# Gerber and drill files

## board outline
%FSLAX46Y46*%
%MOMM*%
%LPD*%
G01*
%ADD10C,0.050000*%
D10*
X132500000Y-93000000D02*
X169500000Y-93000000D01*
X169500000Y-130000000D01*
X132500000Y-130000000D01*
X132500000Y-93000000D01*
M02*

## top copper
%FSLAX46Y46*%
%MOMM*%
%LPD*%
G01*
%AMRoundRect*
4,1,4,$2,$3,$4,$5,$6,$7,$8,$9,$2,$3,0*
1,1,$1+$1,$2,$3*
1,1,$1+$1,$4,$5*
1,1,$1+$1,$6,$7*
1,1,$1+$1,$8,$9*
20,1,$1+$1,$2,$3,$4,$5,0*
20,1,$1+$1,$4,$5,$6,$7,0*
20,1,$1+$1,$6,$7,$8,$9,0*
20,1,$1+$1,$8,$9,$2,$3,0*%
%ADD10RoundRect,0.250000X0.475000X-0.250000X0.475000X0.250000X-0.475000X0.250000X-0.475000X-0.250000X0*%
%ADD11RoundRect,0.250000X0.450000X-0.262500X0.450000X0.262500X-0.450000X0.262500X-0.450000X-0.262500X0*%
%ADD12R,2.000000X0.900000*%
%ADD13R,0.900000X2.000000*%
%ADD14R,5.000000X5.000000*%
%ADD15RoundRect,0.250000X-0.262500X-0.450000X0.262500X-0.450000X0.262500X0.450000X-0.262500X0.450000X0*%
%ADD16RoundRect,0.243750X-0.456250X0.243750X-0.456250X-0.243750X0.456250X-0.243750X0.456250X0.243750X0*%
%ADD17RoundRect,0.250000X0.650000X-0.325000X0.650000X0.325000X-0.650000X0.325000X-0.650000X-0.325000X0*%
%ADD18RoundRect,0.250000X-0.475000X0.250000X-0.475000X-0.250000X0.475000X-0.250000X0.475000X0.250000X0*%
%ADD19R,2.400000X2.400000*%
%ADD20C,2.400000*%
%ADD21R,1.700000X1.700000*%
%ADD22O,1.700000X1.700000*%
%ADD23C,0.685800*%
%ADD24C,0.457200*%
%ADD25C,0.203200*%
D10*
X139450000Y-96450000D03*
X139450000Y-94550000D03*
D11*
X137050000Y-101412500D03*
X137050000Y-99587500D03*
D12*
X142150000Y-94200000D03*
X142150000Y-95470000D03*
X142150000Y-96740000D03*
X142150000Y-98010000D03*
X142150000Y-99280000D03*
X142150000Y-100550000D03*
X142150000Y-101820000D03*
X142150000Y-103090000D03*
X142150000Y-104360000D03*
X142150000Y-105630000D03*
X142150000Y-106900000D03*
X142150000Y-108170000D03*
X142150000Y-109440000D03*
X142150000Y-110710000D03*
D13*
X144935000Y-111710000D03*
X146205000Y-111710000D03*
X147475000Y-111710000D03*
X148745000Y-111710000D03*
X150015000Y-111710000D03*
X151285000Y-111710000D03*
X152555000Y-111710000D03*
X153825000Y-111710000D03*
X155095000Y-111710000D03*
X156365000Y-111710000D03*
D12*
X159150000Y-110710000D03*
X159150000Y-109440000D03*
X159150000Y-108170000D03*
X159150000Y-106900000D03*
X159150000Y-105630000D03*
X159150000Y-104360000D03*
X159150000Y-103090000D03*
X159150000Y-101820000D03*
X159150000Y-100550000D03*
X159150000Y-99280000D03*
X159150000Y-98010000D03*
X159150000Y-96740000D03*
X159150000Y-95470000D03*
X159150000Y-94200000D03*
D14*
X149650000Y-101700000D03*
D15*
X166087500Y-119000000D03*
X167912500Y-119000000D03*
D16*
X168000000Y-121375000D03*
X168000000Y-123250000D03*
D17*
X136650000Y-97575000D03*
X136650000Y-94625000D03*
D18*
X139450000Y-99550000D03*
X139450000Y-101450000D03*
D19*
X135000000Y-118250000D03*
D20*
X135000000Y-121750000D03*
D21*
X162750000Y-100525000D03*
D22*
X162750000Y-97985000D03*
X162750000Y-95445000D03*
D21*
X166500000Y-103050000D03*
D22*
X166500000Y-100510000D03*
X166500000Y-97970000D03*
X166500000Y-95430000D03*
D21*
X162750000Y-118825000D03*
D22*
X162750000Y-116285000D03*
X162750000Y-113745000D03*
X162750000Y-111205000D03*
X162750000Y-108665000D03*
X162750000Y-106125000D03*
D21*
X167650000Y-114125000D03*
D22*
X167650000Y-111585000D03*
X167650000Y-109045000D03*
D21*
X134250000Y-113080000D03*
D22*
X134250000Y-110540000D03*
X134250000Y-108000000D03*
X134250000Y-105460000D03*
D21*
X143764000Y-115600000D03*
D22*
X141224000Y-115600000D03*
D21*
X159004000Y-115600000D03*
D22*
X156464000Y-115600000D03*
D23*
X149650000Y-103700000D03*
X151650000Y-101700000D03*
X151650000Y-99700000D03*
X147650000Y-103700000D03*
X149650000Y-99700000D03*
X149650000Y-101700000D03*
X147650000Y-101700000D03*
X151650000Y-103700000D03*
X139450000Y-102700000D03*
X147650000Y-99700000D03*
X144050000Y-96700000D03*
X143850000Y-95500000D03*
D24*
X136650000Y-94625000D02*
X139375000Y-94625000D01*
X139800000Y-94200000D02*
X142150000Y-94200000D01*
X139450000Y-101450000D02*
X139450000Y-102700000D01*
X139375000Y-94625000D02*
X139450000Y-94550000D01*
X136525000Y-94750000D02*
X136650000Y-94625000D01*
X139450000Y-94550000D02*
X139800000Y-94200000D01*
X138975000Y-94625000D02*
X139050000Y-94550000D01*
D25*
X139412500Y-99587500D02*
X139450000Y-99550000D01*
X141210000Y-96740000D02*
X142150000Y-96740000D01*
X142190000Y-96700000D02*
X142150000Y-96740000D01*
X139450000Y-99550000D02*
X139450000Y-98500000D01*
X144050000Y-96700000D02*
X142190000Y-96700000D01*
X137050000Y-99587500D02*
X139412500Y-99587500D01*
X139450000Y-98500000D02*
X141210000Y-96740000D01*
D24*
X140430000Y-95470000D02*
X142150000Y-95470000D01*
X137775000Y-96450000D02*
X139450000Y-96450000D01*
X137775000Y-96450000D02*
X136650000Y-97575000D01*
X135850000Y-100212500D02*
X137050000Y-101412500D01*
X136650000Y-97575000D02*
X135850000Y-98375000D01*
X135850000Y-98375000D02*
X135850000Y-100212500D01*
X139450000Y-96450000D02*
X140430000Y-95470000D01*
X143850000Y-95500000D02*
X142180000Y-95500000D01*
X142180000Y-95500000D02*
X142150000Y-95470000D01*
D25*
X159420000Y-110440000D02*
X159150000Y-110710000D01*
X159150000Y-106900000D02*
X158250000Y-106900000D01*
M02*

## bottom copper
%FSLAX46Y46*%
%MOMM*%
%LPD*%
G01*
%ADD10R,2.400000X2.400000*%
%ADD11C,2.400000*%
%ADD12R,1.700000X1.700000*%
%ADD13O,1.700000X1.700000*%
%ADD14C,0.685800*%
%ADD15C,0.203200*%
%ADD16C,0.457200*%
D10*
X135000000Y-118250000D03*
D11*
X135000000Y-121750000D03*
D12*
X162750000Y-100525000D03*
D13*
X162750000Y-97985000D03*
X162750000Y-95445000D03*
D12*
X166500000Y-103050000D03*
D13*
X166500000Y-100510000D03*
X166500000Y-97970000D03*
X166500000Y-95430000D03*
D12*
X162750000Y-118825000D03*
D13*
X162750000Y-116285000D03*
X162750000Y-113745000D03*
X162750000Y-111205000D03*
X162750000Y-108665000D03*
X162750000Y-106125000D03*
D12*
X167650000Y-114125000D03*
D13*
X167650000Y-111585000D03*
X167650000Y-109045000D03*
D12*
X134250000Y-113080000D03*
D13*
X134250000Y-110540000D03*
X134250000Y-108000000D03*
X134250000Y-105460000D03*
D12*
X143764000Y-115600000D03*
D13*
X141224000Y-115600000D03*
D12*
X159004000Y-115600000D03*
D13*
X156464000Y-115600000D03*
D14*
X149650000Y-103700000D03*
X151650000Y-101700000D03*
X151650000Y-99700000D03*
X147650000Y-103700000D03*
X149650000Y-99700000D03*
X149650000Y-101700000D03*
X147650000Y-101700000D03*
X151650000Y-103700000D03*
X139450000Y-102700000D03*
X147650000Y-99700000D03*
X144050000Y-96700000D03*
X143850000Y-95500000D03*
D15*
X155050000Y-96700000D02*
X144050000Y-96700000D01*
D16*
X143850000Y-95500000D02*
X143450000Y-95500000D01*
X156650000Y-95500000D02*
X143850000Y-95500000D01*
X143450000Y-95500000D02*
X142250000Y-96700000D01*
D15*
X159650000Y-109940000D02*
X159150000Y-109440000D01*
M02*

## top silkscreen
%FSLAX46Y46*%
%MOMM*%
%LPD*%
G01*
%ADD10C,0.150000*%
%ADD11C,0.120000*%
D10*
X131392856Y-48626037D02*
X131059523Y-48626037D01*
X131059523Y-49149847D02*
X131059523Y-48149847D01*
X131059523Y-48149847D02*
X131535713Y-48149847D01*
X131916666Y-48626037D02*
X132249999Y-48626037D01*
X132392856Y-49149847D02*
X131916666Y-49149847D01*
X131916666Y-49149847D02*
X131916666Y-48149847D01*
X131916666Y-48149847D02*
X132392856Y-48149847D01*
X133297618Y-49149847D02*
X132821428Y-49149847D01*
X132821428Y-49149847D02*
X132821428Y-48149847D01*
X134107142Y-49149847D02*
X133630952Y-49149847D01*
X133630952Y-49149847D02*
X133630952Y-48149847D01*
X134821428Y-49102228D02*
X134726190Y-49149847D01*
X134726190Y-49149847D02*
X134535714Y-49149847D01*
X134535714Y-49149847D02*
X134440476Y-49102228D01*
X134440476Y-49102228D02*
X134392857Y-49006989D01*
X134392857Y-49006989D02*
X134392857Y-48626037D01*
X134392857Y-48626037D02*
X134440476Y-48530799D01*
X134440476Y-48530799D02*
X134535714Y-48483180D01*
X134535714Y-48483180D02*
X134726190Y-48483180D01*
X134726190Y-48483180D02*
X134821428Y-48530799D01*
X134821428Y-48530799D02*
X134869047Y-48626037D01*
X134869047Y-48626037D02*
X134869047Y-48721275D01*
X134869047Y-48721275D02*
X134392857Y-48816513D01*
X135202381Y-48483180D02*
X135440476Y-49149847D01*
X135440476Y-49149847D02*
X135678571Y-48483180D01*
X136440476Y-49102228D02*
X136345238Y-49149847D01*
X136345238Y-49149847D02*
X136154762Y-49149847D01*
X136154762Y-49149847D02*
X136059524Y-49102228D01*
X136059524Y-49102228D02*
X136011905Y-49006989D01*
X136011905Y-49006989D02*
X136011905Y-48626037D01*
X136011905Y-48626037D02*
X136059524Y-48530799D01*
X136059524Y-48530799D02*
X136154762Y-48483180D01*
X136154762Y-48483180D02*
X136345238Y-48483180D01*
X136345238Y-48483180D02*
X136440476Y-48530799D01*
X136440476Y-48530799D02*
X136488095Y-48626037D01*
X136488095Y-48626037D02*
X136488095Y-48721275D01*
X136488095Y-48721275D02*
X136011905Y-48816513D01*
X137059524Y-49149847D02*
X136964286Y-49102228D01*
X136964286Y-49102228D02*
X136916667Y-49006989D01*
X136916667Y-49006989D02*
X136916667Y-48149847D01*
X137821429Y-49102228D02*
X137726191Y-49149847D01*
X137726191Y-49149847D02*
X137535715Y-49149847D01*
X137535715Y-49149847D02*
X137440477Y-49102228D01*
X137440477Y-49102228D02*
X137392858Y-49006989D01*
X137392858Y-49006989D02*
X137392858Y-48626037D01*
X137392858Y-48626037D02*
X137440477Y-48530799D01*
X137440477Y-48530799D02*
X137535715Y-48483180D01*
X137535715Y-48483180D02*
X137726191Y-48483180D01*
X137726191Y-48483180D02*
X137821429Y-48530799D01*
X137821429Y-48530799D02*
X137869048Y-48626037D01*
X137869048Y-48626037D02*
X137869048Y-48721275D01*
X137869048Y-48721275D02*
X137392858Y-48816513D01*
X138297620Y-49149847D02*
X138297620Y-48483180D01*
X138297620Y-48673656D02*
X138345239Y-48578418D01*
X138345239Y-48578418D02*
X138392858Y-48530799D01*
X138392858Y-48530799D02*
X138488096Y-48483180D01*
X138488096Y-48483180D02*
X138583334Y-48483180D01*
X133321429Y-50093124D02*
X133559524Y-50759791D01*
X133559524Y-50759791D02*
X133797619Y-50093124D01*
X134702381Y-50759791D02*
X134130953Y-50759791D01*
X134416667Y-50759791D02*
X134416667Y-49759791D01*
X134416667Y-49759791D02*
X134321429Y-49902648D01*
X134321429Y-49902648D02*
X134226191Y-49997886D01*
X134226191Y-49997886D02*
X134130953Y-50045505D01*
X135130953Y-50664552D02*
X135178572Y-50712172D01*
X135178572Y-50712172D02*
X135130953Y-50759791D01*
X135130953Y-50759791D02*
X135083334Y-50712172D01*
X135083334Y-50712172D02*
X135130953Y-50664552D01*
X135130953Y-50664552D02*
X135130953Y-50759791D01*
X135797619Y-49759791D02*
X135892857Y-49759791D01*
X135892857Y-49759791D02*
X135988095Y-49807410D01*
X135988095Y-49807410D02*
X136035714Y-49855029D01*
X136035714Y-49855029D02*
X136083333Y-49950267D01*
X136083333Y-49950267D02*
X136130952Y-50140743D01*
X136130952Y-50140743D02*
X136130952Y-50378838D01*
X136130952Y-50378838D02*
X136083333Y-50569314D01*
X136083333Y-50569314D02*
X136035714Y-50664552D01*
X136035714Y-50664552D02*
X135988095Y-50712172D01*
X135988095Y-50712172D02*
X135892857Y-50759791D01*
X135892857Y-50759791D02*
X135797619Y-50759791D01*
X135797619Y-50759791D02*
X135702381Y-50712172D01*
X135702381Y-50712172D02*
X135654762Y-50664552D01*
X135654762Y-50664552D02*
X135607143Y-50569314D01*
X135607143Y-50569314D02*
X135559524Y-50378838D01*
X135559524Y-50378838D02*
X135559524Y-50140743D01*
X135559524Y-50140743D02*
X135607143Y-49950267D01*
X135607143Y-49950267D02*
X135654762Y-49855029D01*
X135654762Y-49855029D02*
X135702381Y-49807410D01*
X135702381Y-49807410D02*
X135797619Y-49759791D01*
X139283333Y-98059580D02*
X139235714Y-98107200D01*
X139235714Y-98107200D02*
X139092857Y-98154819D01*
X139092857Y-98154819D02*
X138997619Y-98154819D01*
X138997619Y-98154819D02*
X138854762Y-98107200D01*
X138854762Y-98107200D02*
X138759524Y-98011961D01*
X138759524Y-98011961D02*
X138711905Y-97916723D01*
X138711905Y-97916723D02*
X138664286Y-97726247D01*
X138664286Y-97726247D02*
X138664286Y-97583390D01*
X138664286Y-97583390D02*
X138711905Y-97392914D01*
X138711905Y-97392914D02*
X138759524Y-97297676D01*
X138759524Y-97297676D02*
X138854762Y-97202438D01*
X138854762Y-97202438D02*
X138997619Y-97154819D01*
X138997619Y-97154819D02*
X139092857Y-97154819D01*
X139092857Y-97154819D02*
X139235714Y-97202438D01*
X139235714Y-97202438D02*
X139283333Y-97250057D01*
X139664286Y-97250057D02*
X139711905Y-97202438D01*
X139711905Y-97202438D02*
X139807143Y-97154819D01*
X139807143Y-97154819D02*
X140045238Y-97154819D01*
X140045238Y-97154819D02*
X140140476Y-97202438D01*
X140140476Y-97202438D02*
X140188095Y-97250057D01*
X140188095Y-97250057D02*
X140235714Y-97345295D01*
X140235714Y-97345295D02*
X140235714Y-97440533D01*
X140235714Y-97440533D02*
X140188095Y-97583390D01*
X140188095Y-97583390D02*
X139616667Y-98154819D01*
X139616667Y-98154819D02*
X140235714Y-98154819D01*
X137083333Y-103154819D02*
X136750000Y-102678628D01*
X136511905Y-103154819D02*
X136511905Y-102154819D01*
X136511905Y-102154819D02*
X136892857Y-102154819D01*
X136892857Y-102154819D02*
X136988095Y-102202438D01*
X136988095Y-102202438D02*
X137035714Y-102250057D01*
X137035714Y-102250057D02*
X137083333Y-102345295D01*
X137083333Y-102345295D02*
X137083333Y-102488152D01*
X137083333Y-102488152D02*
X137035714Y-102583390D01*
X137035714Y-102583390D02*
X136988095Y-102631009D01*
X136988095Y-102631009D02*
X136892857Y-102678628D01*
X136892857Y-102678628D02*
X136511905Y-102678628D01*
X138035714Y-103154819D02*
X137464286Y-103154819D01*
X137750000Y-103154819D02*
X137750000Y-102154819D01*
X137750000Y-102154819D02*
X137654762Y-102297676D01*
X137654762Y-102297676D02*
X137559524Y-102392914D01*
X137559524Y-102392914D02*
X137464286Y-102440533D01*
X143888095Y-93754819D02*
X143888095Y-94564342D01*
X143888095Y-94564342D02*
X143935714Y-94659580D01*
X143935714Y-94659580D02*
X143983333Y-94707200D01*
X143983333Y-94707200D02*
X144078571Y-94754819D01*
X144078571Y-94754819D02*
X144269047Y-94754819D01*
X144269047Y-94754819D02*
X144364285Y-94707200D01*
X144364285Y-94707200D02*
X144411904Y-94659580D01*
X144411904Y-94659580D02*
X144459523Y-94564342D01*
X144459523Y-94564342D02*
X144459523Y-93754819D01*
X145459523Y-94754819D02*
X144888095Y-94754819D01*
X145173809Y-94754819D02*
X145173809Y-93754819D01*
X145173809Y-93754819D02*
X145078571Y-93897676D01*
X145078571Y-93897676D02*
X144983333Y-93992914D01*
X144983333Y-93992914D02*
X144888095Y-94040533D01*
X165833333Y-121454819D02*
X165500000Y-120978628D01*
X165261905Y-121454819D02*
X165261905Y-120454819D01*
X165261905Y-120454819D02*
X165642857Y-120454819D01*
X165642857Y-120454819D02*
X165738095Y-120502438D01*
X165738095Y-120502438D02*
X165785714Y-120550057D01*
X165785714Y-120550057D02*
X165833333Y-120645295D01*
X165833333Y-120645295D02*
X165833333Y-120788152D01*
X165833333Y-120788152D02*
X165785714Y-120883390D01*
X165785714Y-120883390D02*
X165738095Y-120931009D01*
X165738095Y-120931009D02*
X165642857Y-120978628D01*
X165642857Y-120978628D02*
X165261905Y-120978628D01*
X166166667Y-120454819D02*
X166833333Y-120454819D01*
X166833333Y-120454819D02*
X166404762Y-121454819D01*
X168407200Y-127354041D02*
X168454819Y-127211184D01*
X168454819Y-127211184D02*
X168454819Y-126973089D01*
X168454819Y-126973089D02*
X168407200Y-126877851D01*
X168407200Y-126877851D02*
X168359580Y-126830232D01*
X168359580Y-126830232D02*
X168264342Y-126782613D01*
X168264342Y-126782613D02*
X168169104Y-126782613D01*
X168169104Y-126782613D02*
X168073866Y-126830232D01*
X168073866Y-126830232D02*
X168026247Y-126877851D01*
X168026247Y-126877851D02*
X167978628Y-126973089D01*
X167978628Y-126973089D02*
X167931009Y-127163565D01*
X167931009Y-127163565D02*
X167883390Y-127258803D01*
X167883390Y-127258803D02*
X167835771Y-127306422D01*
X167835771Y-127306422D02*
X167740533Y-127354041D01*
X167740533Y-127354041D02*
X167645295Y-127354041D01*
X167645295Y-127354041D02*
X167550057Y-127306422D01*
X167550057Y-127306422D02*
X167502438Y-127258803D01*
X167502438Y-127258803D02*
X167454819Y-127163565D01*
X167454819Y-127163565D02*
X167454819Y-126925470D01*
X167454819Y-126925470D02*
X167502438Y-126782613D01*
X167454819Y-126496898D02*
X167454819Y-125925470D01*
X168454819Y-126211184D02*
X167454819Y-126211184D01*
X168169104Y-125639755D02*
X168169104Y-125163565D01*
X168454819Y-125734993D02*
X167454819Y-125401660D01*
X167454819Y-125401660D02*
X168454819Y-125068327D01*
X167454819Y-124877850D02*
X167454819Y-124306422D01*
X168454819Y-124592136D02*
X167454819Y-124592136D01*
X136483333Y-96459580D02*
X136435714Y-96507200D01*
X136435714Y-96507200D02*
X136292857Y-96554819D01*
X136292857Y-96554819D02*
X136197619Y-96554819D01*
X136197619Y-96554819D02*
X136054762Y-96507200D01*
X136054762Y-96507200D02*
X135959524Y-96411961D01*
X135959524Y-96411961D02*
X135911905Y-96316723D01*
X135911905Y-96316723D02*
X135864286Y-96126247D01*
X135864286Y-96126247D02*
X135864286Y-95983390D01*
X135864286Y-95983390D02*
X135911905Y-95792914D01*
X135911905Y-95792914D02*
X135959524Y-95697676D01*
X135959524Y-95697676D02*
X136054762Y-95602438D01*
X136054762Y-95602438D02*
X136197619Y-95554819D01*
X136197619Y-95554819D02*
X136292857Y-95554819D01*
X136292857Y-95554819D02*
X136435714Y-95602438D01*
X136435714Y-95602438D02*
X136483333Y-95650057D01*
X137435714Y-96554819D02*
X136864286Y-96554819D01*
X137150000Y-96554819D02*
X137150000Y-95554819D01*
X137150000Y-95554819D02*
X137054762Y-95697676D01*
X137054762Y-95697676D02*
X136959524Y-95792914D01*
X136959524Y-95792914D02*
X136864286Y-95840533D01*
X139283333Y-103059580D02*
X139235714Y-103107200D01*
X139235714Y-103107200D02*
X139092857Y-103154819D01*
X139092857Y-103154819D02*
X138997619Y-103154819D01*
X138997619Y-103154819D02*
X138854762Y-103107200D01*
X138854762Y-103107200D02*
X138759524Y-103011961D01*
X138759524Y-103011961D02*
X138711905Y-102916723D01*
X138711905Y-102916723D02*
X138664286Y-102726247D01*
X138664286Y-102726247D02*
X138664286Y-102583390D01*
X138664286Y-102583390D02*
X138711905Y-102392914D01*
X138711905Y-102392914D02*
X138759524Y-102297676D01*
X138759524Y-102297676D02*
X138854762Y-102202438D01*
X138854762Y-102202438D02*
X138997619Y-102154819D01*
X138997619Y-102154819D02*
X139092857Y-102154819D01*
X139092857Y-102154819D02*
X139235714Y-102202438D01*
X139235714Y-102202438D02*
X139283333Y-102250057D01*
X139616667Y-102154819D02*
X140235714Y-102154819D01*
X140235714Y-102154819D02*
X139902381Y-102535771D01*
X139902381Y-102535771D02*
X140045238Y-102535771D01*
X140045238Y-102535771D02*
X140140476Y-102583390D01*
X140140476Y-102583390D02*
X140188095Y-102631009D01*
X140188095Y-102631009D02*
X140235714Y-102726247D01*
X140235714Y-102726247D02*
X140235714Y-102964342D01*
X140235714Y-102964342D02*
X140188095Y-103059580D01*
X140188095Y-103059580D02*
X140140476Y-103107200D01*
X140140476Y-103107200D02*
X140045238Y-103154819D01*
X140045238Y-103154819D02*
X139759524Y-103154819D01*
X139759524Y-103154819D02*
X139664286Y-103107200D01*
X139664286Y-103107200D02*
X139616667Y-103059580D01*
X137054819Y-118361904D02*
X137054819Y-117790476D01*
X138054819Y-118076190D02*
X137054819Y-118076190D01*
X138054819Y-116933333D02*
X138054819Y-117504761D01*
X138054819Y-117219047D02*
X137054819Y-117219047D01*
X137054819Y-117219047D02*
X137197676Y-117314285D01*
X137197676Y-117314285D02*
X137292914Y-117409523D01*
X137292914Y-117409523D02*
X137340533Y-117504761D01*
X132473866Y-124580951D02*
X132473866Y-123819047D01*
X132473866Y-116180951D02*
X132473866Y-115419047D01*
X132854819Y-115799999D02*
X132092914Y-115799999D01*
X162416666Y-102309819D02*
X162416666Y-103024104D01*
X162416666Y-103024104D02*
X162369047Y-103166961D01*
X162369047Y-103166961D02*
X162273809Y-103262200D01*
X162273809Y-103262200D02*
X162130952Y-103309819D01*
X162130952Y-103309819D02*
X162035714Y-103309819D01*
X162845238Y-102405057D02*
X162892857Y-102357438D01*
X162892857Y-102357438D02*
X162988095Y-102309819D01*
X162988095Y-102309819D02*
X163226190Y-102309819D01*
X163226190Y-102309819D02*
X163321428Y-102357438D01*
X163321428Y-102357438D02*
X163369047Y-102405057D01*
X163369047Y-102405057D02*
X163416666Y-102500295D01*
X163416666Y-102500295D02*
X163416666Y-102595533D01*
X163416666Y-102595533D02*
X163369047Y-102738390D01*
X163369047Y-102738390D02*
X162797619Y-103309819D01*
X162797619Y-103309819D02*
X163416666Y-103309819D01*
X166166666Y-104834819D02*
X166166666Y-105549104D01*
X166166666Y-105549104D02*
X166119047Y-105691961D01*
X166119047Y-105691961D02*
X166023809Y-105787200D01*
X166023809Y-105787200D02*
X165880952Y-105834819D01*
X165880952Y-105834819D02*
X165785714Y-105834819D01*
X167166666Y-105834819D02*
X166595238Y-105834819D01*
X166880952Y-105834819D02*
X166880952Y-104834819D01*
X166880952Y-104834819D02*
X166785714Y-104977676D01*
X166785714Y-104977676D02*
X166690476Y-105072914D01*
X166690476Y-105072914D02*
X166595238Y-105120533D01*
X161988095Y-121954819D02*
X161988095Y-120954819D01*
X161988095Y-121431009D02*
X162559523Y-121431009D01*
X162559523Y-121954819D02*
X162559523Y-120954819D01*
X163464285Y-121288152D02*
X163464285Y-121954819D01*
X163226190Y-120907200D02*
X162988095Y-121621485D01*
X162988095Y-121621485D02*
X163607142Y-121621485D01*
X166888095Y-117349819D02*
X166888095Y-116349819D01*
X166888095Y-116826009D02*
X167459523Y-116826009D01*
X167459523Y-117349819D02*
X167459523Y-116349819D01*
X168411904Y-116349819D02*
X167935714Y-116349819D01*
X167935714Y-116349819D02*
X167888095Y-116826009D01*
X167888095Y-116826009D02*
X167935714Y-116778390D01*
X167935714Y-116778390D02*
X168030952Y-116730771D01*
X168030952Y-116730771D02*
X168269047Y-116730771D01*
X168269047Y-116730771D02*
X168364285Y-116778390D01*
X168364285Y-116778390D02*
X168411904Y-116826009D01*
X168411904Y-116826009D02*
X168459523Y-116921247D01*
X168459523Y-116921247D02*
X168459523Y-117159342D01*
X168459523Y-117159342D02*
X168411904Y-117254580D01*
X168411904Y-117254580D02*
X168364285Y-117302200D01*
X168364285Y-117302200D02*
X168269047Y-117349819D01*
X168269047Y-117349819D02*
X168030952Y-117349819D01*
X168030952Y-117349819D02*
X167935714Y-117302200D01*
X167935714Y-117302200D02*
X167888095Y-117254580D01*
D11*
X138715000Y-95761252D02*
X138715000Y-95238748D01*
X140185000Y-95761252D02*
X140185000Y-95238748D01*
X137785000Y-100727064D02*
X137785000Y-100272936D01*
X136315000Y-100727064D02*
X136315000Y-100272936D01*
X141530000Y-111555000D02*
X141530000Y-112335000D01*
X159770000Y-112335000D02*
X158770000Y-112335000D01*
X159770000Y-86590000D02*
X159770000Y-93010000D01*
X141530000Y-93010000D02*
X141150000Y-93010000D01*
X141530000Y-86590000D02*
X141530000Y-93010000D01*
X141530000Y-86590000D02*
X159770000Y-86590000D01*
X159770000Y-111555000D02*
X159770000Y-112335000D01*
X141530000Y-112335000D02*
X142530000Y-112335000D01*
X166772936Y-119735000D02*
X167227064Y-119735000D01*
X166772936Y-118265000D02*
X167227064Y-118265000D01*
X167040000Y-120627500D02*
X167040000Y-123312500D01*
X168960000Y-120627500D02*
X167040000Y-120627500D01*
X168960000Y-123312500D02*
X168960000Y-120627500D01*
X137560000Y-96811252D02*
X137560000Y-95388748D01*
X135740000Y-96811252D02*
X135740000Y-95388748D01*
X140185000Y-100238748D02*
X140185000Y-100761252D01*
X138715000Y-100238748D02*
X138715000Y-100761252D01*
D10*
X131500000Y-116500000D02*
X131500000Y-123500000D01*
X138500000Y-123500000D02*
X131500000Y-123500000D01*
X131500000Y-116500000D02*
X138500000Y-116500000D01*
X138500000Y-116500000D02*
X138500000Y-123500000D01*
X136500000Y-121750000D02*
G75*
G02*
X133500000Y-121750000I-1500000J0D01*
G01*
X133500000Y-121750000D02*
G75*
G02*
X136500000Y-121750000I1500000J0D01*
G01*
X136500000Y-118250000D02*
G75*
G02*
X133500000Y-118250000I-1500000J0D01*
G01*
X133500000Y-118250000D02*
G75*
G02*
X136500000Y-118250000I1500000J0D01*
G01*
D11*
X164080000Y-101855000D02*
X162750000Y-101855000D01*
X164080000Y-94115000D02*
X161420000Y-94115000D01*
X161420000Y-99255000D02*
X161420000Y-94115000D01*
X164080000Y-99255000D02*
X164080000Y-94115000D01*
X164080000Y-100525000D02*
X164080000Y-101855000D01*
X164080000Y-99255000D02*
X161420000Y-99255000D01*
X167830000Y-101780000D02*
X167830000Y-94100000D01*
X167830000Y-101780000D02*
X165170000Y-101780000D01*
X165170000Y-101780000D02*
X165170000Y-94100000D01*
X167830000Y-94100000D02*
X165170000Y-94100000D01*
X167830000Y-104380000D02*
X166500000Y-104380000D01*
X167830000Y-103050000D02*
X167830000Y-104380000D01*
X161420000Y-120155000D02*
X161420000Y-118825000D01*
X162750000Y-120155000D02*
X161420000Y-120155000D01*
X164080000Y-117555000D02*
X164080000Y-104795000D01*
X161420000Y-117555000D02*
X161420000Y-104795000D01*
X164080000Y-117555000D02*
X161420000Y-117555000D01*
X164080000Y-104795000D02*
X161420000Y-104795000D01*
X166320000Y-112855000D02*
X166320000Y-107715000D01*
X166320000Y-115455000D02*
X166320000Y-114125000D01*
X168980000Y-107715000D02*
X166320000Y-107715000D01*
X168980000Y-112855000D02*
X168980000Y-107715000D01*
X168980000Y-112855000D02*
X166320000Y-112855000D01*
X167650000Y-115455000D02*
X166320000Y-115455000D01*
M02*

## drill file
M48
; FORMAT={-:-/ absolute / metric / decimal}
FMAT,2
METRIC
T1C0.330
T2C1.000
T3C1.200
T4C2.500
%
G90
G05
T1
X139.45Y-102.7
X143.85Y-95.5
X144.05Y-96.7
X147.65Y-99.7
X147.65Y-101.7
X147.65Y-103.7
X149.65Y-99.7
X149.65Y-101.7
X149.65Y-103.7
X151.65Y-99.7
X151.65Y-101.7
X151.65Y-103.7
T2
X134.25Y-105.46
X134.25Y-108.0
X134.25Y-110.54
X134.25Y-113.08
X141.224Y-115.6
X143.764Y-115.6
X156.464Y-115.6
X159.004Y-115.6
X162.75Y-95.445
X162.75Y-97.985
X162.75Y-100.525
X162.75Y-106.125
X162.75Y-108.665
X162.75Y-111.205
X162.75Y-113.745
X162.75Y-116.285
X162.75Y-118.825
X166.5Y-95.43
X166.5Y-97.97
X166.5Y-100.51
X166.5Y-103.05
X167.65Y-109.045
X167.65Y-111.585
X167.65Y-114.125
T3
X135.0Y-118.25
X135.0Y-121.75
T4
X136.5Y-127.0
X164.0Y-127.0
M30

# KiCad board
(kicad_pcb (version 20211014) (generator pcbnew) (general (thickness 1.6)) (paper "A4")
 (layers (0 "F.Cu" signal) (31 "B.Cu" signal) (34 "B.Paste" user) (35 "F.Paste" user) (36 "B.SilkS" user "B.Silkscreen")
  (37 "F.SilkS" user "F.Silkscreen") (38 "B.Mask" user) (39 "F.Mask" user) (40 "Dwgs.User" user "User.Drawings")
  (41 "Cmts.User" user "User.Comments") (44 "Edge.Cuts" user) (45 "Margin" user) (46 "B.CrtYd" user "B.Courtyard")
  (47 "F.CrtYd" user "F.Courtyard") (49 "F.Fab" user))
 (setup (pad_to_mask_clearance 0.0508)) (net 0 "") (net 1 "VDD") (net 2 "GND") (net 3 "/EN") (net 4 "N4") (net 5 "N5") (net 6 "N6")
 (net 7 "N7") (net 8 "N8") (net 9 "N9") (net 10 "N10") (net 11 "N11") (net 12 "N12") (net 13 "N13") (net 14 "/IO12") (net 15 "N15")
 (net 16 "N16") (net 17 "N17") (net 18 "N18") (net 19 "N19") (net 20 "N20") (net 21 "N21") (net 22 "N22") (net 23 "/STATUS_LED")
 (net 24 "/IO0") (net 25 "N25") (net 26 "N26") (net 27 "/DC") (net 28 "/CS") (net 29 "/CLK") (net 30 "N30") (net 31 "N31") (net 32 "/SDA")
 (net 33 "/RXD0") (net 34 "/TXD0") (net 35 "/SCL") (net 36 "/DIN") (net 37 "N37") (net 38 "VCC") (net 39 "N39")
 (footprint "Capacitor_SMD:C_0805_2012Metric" (layer "F.Cu") (at 139.45 95.5 90)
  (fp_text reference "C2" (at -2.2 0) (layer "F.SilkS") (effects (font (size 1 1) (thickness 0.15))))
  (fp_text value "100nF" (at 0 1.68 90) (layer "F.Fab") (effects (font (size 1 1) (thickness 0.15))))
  (fp_line (start -0.261252 -0.735) (end 0.261252 -0.735) (layer "F.SilkS") (width 0.12))
  (fp_line (start -0.261252 0.735) (end 0.261252 0.735) (layer "F.SilkS") (width 0.12))
  (pad "1" smd roundrect locked (at -0.95 0 90) (size 1 1.45) (layers "F.Cu" "F.Paste" "F.Mask") (roundrect_rratio 0.25) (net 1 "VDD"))
  (pad "2" smd roundrect locked (at 0.95 0 90) (size 1 1.45) (layers "F.Cu" "F.Paste" "F.Mask") (roundrect_rratio 0.25) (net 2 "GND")))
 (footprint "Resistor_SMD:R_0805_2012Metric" (layer "F.Cu") (at 137.05 100.5 90)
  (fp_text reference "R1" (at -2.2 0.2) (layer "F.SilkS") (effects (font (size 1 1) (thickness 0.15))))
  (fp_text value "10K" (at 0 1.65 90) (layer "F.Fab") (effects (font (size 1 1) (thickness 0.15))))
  (fp_line (start -0.227064 0.735) (end 0.227064 0.735) (layer "F.SilkS") (width 0.12))
  (fp_line (start -0.227064 -0.735) (end 0.227064 -0.735) (layer "F.SilkS") (width 0.12))
  (pad "1" smd roundrect locked (at -0.9125 0 90) (size 1.025 1.4) (layers "F.Cu" "F.Paste" "F.Mask") (roundrect_rratio 0.243902)
   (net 1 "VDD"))
  (pad "2" smd roundrect locked (at 0.9125 0 90) (size 1.025 1.4) (layers "F.Cu" "F.Paste" "F.Mask") (roundrect_rratio 0.243902)
   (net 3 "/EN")))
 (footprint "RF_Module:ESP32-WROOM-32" (layer "F.Cu") (at 150.65 102.455)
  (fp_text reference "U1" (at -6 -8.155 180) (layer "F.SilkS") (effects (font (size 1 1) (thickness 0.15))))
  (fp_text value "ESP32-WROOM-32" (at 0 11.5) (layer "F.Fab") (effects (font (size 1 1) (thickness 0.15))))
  (fp_line (start -9.12 9.1) (end -9.12 9.88) (layer "F.SilkS") (width 0.12))
  (fp_line (start 9.12 9.88) (end 8.12 9.88) (layer "F.SilkS") (width 0.12))
  (fp_line (start 9.12 -15.865) (end 9.12 -9.445) (layer "F.SilkS") (width 0.12))
  (fp_line (start -9.12 -9.445) (end -9.5 -9.445) (layer "F.SilkS") (width 0.12))
  (fp_line (start -9.12 -15.865) (end -9.12 -9.445) (layer "F.SilkS") (width 0.12))
  (fp_line (start -9.12 -15.865) (end 9.12 -15.865) (layer "F.SilkS") (width 0.12))
  (fp_line (start 9.12 9.1) (end 9.12 9.88) (layer "F.SilkS") (width 0.12))
  (fp_line (start -9.12 9.88) (end -8.12 9.88) (layer "F.SilkS") (width 0.12))
  (pad "1" smd rect locked (at -8.5 -8.255) (size 2 0.9) (layers "F.Cu" "F.Paste" "F.Mask") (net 2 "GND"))
  (pad "2" smd rect locked (at -8.5 -6.985) (size 2 0.9) (layers "F.Cu" "F.Paste" "F.Mask") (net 1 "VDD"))
  (pad "3" smd rect locked (at -8.5 -5.715) (size 2 0.9) (layers "F.Cu" "F.Paste" "F.Mask") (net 3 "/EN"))
  (pad "4" smd rect locked (at -8.5 -4.445) (size 2 0.9) (layers "F.Cu" "F.Paste" "F.Mask") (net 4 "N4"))
  (pad "5" smd rect locked (at -8.5 -3.175) (size 2 0.9) (layers "F.Cu" "F.Paste" "F.Mask") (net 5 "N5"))
  (pad "6" smd rect locked (at -8.5 -1.905) (size 2 0.9) (layers "F.Cu" "F.Paste" "F.Mask") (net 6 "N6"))
  (pad "7" smd rect locked (at -8.5 -0.635) (size 2 0.9) (layers "F.Cu" "F.Paste" "F.Mask") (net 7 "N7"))
  (pad "8" smd rect locked (at -8.5 0.635) (size 2 0.9) (layers "F.Cu" "F.Paste" "F.Mask") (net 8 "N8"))
  (pad "9" smd rect locked (at -8.5 1.905) (size 2 0.9) (layers "F.Cu" "F.Paste" "F.Mask") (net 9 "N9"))
  (pad "10" smd rect locked (at -8.5 3.175) (size 2 0.9) (layers "F.Cu" "F.Paste" "F.Mask") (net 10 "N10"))
  (pad "11" smd rect locked (at -8.5 4.445) (size 2 0.9) (layers "F.Cu" "F.Paste" "F.Mask") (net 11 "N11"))
  (pad "12" smd rect locked (at -8.5 5.715) (size 2 0.9) (layers "F.Cu" "F.Paste" "F.Mask") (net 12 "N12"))
  (pad "13" smd rect locked (at -8.5 6.985) (size 2 0.9) (layers "F.Cu" "F.Paste" "F.Mask") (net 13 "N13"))
  (pad "14" smd rect locked (at -8.5 8.255) (size 2 0.9) (layers "F.Cu" "F.Paste" "F.Mask") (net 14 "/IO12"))
  (pad "15" smd rect locked (at -5.715 9.255 90) (size 2 0.9) (layers "F.Cu" "F.Paste" "F.Mask") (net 2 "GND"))
  (pad "16" smd rect locked (at -4.445 9.255 90) (size 2 0.9) (layers "F.Cu" "F.Paste" "F.Mask") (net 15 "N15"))
  (pad "17" smd rect locked (at -3.175 9.255 90) (size 2 0.9) (layers "F.Cu" "F.Paste" "F.Mask") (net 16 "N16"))
  (pad "18" smd rect locked (at -1.905 9.255 90) (size 2 0.9) (layers "F.Cu" "F.Paste" "F.Mask") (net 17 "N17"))
  (pad "19" smd rect locked (at -0.635 9.255 90) (size 2 0.9) (layers "F.Cu" "F.Paste" "F.Mask") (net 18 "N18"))
  (pad "20" smd rect locked (at 0.635 9.255 90) (size 2 0.9) (layers "F.Cu" "F.Paste" "F.Mask") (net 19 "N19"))
  (pad "21" smd rect locked (at 1.905 9.255 90) (size 2 0.9) (layers "F.Cu" "F.Paste" "F.Mask") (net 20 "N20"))
  (pad "22" smd rect locked (at 3.175 9.255 90) (size 2 0.9) (layers "F.Cu" "F.Paste" "F.Mask") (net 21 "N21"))
  (pad "23" smd rect locked (at 4.445 9.255 90) (size 2 0.9) (layers "F.Cu" "F.Paste" "F.Mask") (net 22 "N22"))
  (pad "24" smd rect locked (at 5.715 9.255 90) (size 2 0.9) (layers "F.Cu" "F.Paste" "F.Mask") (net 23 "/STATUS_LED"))
  (pad "25" smd rect locked (at 8.5 8.255) (size 2 0.9) (layers "F.Cu" "F.Paste" "F.Mask") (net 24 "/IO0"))
  (pad "26" smd rect locked (at 8.5 6.985) (size 2 0.9) (layers "F.Cu" "F.Paste" "F.Mask") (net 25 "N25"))
  (pad "27" smd rect locked (at 8.5 5.715) (size 2 0.9) (layers "F.Cu" "F.Paste" "F.Mask") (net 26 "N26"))
  (pad "28" smd rect locked (at 8.5 4.445) (size 2 0.9) (layers "F.Cu" "F.Paste" "F.Mask") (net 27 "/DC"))
  (pad "29" smd rect locked (at 8.5 3.175) (size 2 0.9) (layers "F.Cu" "F.Paste" "F.Mask") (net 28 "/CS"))
  (pad "30" smd rect locked (at 8.5 1.905) (size 2 0.9) (layers "F.Cu" "F.Paste" "F.Mask") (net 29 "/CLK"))
  (pad "31" smd rect locked (at 8.5 0.635) (size 2 0.9) (layers "F.Cu" "F.Paste" "F.Mask") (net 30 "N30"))
  (pad "32" smd rect locked (at 8.5 -0.635) (size 2 0.9) (layers "F.Cu" "F.Paste" "F.Mask") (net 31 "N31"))
  (pad "33" smd rect locked (at 8.5 -1.905) (size 2 0.9) (layers "F.Cu" "F.Paste" "F.Mask") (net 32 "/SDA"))
  (pad "34" smd rect locked (at 8.5 -3.175) (size 2 0.9) (layers "F.Cu" "F.Paste" "F.Mask") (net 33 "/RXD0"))
  (pad "35" smd rect locked (at 8.5 -4.445) (size 2 0.9) (layers "F.Cu" "F.Paste" "F.Mask") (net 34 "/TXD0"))
  (pad "36" smd rect locked (at 8.5 -5.715) (size 2 0.9) (layers "F.Cu" "F.Paste" "F.Mask") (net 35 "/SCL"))
  (pad "37" smd rect locked (at 8.5 -6.985) (size 2 0.9) (layers "F.Cu" "F.Paste" "F.Mask") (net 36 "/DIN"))
  (pad "38" smd rect locked (at 8.5 -8.255) (size 2 0.9) (layers "F.Cu" "F.Paste" "F.Mask") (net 2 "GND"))
  (pad "39" smd rect locked (at -1 -0.755) (size 5 5) (layers "F.Cu" "F.Paste" "F.Mask") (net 2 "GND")))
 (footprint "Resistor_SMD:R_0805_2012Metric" (layer "F.Cu") (at 167 119)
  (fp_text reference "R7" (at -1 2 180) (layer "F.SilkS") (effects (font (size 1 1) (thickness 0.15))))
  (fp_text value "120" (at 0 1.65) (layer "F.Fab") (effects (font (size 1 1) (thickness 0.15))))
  (fp_line (start -0.227064 0.735) (end 0.227064 0.735) (layer "F.SilkS") (width 0.12))
  (fp_line (start -0.227064 -0.735) (end 0.227064 -0.735) (layer "F.SilkS") (width 0.12))
  (pad "1" smd roundrect locked (at -0.9125 0) (size 1.025 1.4) (layers "F.Cu" "F.Paste" "F.Mask") (roundrect_rratio 0.243902)
   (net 23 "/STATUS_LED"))
  (pad "2" smd roundrect locked (at 0.9125 0) (size 1.025 1.4) (layers "F.Cu" "F.Paste" "F.Mask") (roundrect_rratio 0.243902) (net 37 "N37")))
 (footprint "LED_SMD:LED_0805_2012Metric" (layer "F.Cu") (at 168 122.3125 -90)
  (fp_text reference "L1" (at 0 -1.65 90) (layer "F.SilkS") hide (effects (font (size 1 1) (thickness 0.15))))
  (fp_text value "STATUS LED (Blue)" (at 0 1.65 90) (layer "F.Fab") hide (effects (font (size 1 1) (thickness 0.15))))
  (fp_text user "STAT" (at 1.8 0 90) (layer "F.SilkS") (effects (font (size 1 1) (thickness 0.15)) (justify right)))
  (fp_line (start -1.685 0.96) (end 1 0.96) (layer "F.SilkS") (width 0.12))
  (fp_line (start -1.685 -0.96) (end -1.685 0.96) (layer "F.SilkS") (width 0.12))
  (fp_line (start 1 -0.96) (end -1.685 -0.96) (layer "F.SilkS") (width 0.12))
  (pad "1" smd roundrect locked (at -0.9375 0 270) (size 0.975 1.4) (layers "F.Cu" "F.Paste" "F.Mask") (roundrect_rratio 0.25)
   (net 37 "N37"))
  (pad "2" smd roundrect locked (at 0.9375 0 270) (size 0.975 1.4) (layers "F.Cu" "F.Paste" "F.Mask") (roundrect_rratio 0.25) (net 1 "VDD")))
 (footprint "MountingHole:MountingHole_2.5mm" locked (layer "F.Cu") (at 136.5 127)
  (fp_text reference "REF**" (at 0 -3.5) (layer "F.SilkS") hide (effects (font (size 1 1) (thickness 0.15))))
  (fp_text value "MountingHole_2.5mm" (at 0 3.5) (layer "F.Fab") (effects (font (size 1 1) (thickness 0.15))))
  (pad "" np_thru_hole circle locked (at 0 0) (size 2.5 2.5) (drill 2.5) (layers *.Cu *.Mask)))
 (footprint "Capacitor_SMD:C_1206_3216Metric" (layer "F.Cu") (at 136.65 96.1 90)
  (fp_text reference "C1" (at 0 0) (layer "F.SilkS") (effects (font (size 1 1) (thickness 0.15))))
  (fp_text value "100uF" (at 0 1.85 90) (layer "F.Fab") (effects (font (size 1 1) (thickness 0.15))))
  (fp_line (start -0.711252 0.91) (end 0.711252 0.91) (layer "F.SilkS") (width 0.12))
  (fp_line (start -0.711252 -0.91) (end 0.711252 -0.91) (layer "F.SilkS") (width 0.12))
  (pad "1" smd roundrect locked (at -1.475 0 90) (size 1.15 1.8) (layers "F.Cu" "F.Paste" "F.Mask") (roundrect_rratio 0.217391)
   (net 1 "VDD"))
  (pad "2" smd roundrect locked (at 1.475 0 90) (size 1.15 1.8) (layers "F.Cu" "F.Paste" "F.Mask") (roundrect_rratio 0.217391) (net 2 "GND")))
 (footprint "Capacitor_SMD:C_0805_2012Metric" (layer "F.Cu") (at 139.45 100.5 -90)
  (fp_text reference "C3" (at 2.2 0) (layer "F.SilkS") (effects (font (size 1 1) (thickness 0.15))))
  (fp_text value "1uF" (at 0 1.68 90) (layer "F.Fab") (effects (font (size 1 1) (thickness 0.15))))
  (fp_line (start -0.261252 -0.735) (end 0.261252 -0.735) (layer "F.SilkS") (width 0.12))
  (fp_line (start -0.261252 0.735) (end 0.261252 0.735) (layer "F.SilkS") (width 0.12))
  (pad "1" smd roundrect locked (at -0.95 0 270) (size 1 1.45) (layers "F.Cu" "F.Paste" "F.Mask") (roundrect_rratio 0.25) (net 3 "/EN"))
  (pad "2" smd roundrect locked (at 0.95 0 270) (size 1 1.45) (layers "F.Cu" "F.Paste" "F.Mask") (roundrect_rratio 0.25) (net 2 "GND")))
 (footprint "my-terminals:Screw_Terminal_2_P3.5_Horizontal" (layer "F.Cu") (at 135 120 -90)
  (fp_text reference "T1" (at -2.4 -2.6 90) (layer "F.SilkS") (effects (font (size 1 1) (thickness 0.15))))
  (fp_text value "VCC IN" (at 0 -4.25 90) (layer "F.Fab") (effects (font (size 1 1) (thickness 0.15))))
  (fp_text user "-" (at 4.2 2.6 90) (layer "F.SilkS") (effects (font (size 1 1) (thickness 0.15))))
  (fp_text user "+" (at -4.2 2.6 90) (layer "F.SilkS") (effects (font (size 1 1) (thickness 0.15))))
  (fp_line (start -3.5 3.5) (end 3.5 3.5) (layer "F.SilkS") (width 0.15))
  (fp_line (start 3.5 -3.5) (end 3.5 3.5) (layer "F.SilkS") (width 0.15))
  (fp_line (start -3.5 3.5) (end -3.5 -3.5) (layer "F.SilkS") (width 0.15))
  (fp_line (start -3.5 -3.5) (end 3.5 -3.5) (layer "F.SilkS") (width 0.15))
  (fp_circle (center 1.75 0) (end 3.25 0) (layer "F.SilkS") (width 0.15) (fill none))
  (fp_circle (center -1.75 0) (end -0.25 0) (layer "F.SilkS") (width 0.15) (fill none))
  (pad "1" thru_hole rect locked (at -1.75 0 270) (size 2.4 2.4) (drill 1.2) (layers *.Cu *.Mask) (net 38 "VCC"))
  (pad "2" thru_hole circle locked (at 1.75 0 270) (size 2.4 2.4) (drill 1.2) (layers *.Cu *.Mask) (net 2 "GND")))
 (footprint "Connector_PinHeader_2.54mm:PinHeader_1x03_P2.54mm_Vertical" (layer "F.Cu") (at 162.75 100.525 180)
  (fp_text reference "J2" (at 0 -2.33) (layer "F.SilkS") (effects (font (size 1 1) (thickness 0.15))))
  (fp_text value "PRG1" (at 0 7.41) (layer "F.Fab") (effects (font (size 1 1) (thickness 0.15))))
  (fp_line (start -1.33 -1.33) (end 0 -1.33) (layer "F.SilkS") (width 0.12))
  (fp_line (start -1.33 6.41) (end 1.33 6.41) (layer "F.SilkS") (width 0.12))
  (fp_line (start 1.33 1.27) (end 1.33 6.41) (layer "F.SilkS") (width 0.12))
  (fp_line (start -1.33 1.27) (end -1.33 6.41) (layer "F.SilkS") (width 0.12))
  (fp_line (start -1.33 0) (end -1.33 -1.33) (layer "F.SilkS") (width 0.12))
  (fp_line (start -1.33 1.27) (end 1.33 1.27) (layer "F.SilkS") (width 0.12))
  (pad "1" thru_hole rect (at 0 0 180) (size 1.7 1.7) (drill 1) (layers *.Cu *.Mask) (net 3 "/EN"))
  (pad "2" thru_hole oval (at 0 2.54 180) (size 1.7 1.7) (drill 1) (layers *.Cu *.Mask) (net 24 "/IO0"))
  (pad "3" thru_hole oval (at 0 5.08 180) (size 1.7 1.7) (drill 1) (layers *.Cu *.Mask) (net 2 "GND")))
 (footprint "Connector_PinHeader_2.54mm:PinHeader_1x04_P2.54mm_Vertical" (layer "F.Cu") (at 166.5 103.05 180)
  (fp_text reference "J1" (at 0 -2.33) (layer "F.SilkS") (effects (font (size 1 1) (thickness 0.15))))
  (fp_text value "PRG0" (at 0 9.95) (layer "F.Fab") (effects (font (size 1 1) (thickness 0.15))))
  (fp_line (start -1.33 1.27) (end -1.33 8.95) (layer "F.SilkS") (width 0.12))
  (fp_line (start -1.33 1.27) (end 1.33 1.27) (layer "F.SilkS") (width 0.12))
  (fp_line (start 1.33 1.27) (end 1.33 8.95) (layer "F.SilkS") (width 0.12))
  (fp_line (start -1.33 8.95) (end 1.33 8.95) (layer "F.SilkS") (width 0.12))
  (fp_line (start -1.33 -1.33) (end 0 -1.33) (layer "F.SilkS") (width 0.12))
  (fp_line (start -1.33 0) (end -1.33 -1.33) (layer "F.SilkS") (width 0.12))
  (pad "1" thru_hole rect (at 0 0 180) (size 1.7 1.7) (drill 1) (layers *.Cu *.Mask) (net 34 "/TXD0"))
  (pad "2" thru_hole oval (at 0 2.54 180) (size 1.7 1.7) (drill 1) (layers *.Cu *.Mask) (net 33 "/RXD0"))
  (pad "3" thru_hole oval (at 0 5.08 180) (size 1.7 1.7) (drill 1) (layers *.Cu *.Mask) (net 1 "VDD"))
  (pad "4" thru_hole oval (at 0 7.62 180) (size 1.7 1.7) (drill 1) (layers *.Cu *.Mask) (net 2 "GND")))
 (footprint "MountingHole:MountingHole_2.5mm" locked (layer "F.Cu") (at 164 127)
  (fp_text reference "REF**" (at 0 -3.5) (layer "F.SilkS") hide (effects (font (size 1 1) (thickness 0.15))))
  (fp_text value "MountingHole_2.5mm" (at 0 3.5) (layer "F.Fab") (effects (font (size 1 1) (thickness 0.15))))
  (pad "" np_thru_hole circle locked (at 0 0) (size 2.5 2.5) (drill 2.5) (layers *.Cu *.Mask)))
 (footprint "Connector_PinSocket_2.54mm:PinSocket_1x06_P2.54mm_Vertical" (layer "F.Cu") (at 162.75 118.825 180)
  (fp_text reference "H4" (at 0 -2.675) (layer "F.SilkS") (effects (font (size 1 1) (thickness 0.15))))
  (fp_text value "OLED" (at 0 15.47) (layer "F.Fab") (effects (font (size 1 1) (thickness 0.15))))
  (fp_line (start 1.33 -1.33) (end 1.33 0) (layer "F.SilkS") (width 0.12))
  (fp_line (start 0 -1.33) (end 1.33 -1.33) (layer "F.SilkS") (width 0.12))
  (fp_line (start -1.33 1.27) (end -1.33 14.03) (layer "F.SilkS") (width 0.12))
  (fp_line (start 1.33 1.27) (end 1.33 14.03) (layer "F.SilkS") (width 0.12))
  (fp_line (start -1.33 1.27) (end 1.33 1.27) (layer "F.SilkS") (width 0.12))
  (fp_line (start -1.33 14.03) (end 1.33 14.03) (layer "F.SilkS") (width 0.12))
  (pad "1" thru_hole rect (at 0 0 180) (size 1.7 1.7) (drill 1) (layers *.Cu *.Mask) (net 1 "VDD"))
  (pad "2" thru_hole oval (at 0 2.54 180) (size 1.7 1.7) (drill 1) (layers *.Cu *.Mask) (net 2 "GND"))
  (pad "3" thru_hole oval (at 0 5.08 180) (size 1.7 1.7) (drill 1) (layers *.Cu *.Mask) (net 36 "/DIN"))
  (pad "4" thru_hole oval (at 0 7.62 180) (size 1.7 1.7) (drill 1) (layers *.Cu *.Mask) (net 29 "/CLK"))
  (pad "5" thru_hole oval (at 0 10.16 180) (size 1.7 1.7) (drill 1) (layers *.Cu *.Mask) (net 28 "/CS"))
  (pad "6" thru_hole oval (at 0 12.7 180) (size 1.7 1.7) (drill 1) (layers *.Cu *.Mask) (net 27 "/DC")))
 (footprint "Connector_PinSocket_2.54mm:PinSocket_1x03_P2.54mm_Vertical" (layer "F.Cu") (at 167.65 114.125 180)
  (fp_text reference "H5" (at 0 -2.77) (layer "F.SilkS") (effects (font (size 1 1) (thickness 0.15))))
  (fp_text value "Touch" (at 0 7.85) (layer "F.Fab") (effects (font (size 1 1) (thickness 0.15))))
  (fp_line (start 1.33 1.27) (end 1.33 6.41) (layer "F.SilkS") (width 0.12))
  (fp_line (start 1.33 -1.33) (end 1.33 0) (layer "F.SilkS") (width 0.12))
  (fp_line (start -1.33 6.41) (end 1.33 6.41) (layer "F.SilkS") (width 0.12))
  (fp_line (start -1.33 1.27) (end -1.33 6.41) (layer "F.SilkS") (width 0.12))
  (fp_line (start -1.33 1.27) (end 1.33 1.27) (layer "F.SilkS") (width 0.12))
  (fp_line (start 0 -1.33) (end 1.33 -1.33) (layer "F.SilkS") (width 0.12))
  (pad "1" thru_hole rect (at 0 0 180) (size 1.7 1.7) (drill 1) (layers *.Cu *.Mask) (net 2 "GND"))
  (pad "2" thru_hole oval (at 0 2.54 180) (size 1.7 1.7) (drill 1) (layers *.Cu *.Mask) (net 14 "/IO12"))
  (pad "3" thru_hole oval (at 0 5.08 180) (size 1.7 1.7) (drill 1) (layers *.Cu *.Mask) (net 1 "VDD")))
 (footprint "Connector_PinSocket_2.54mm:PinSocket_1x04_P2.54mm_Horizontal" (layer "B.Cu") (at 134.25 113.08)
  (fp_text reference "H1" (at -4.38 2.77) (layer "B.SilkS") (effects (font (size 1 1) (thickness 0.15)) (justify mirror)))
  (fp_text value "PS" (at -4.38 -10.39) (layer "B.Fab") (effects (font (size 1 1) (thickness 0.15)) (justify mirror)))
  (pad "1" thru_hole rect (at 0 0) (size 1.7 1.7) (drill 1) (layers *.Cu *.Mask) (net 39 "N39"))
  (pad "2" thru_hole oval (at 0 -2.54) (size 1.7 1.7) (drill 1) (layers *.Cu *.Mask) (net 38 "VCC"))
  (pad "3" thru_hole oval (at 0 -5.08) (size 1.7 1.7) (drill 1) (layers *.Cu *.Mask) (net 2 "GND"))
  (pad "4" thru_hole oval (at 0 -7.62) (size 1.7 1.7) (drill 1) (layers *.Cu *.Mask) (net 1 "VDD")))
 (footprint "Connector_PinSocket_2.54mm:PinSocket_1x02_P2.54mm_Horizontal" (layer "B.Cu") (at 143.764 115.6 90)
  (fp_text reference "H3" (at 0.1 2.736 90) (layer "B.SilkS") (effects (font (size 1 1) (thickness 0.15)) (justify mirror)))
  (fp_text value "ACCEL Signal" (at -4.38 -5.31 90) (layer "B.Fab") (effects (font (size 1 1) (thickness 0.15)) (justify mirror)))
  (pad "1" thru_hole rect (at 0 0 90) (size 1.7 1.7) (drill 1) (layers *.Cu *.Mask) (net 32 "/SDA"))
  (pad "2" thru_hole oval (at 0 -2.54 90) (size 1.7 1.7) (drill 1) (layers *.Cu *.Mask) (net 35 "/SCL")))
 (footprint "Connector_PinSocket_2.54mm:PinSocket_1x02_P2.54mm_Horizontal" (layer "B.Cu") (at 159.004 115.6 90)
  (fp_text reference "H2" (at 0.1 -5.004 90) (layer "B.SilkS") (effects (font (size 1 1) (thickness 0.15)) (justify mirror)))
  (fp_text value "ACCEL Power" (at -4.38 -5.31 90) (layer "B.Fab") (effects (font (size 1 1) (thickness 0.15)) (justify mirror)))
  (pad "1" thru_hole rect (at 0 0 90) (size 1.7 1.7) (drill 1) (layers *.Cu *.Mask) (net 2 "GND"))
  (pad "2" thru_hole oval (at 0 -2.54 90) (size 1.7 1.7) (drill 1) (layers *.Cu *.Mask) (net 1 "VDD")))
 (gr_rect (start 132.5 93) (end 169.5 130) (layer "Edge.Cuts") (width 0.05) (fill none))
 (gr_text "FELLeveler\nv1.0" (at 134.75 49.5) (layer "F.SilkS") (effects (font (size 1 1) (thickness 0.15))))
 (segment (start 136.65 94.625) (end 139.375 94.625) (width 0.4572) (layer "F.Cu") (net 2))
 (segment (start 139.8 94.2) (end 142.15 94.2) (width 0.4572) (layer "F.Cu") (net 2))
 (segment (start 139.45 101.45) (end 139.45 102.7) (width 0.4572) (layer "F.Cu") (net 2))
 (segment (start 139.375 94.625) (end 139.45 94.55) (width 0.4572) (layer "F.Cu") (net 2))
 (segment (start 136.525 94.75) (end 136.65 94.625) (width 0.4572) (layer "F.Cu") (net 2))
 (segment (start 139.45 94.55) (end 139.8 94.2) (width 0.4572) (layer "F.Cu") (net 2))
 (segment (start 138.975 94.625) (end 139.05 94.55) (width 0.4572) (layer "F.Cu") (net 2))
 (via (at 149.65 103.7) (size 0.6858) (drill 0.3302) (layers "F.Cu" "B.Cu") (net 2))
 (via (at 151.65 101.7) (size 0.6858) (drill 0.3302) (layers "F.Cu" "B.Cu") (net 2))
 (via (at 151.65 99.7) (size 0.6858) (drill 0.3302) (layers "F.Cu" "B.Cu") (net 2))
 (via (at 147.65 103.7) (size 0.6858) (drill 0.3302) (layers "F.Cu" "B.Cu") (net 2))
 (via (at 149.65 99.7) (size 0.6858) (drill 0.3302) (layers "F.Cu" "B.Cu") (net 2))
 (via (at 149.65 101.7) (size 0.6858) (drill 0.3302) (layers "F.Cu" "B.Cu") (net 2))
 (via (at 147.65 101.7) (size 0.6858) (drill 0.3302) (layers "F.Cu" "B.Cu") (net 2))
 (via (at 151.65 103.7) (size 0.6858) (drill 0.3302) (layers "F.Cu" "B.Cu") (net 2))
 (via (at 139.45 102.7) (size 0.6858) (drill 0.3302) (layers "F.Cu" "B.Cu") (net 2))
 (via (at 147.65 99.7) (size 0.6858) (drill 0.3302) (layers "F.Cu" "B.Cu") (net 2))
 (segment (start 139.4125 99.5875) (end 139.45 99.55) (width 0.2032) (layer "F.Cu") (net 3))
 (segment (start 141.21 96.74) (end 142.15 96.74) (width 0.2032) (layer "F.Cu") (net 3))
 (segment (start 142.19 96.7) (end 142.15 96.74) (width 0.2032) (layer "F.Cu") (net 3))
 (segment (start 139.45 99.55) (end 139.45 98.5) (width 0.2032) (layer "F.Cu") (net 3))
 (segment (start 144.05 96.7) (end 142.19 96.7) (width 0.2032) (layer "F.Cu") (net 3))
 (segment (start 137.05 99.5875) (end 139.4125 99.5875) (width 0.2032) (layer "F.Cu") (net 3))
 (segment (start 139.45 98.5) (end 141.21 96.74) (width 0.2032) (layer "F.Cu") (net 3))
 (via (at 144.05 96.7) (size 0.6858) (drill 0.3302) (layers "F.Cu" "B.Cu") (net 3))
 (segment (start 155.05 96.7) (end 144.05 96.7) (width 0.2032) (layer "B.Cu") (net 3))
 (segment (start 140.43 95.47) (end 142.15 95.47) (width 0.4572) (layer "F.Cu") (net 1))
 (segment (start 137.775 96.45) (end 139.45 96.45) (width 0.4572) (layer "F.Cu") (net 1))
 (segment (start 137.775 96.45) (end 136.65 97.575) (width 0.4572) (layer "F.Cu") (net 1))
 (segment (start 135.85 100.2125) (end 137.05 101.4125) (width 0.4572) (layer "F.Cu") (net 1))
 (segment (start 136.65 97.575) (end 135.85 98.375) (width 0.4572) (layer "F.Cu") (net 1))
 (segment (start 135.85 98.375) (end 135.85 100.2125) (width 0.4572) (layer "F.Cu") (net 1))
 (segment (start 139.45 96.45) (end 140.43 95.47) (width 0.4572) (layer "F.Cu") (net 1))
 (segment (start 143.85 95.5) (end 142.18 95.5) (width 0.4572) (layer "F.Cu") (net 1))
 (segment (start 142.18 95.5) (end 142.15 95.47) (width 0.4572) (layer "F.Cu") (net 1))
 (via (at 143.85 95.5) (size 0.6858) (drill 0.3302) (layers "F.Cu" "B.Cu") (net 1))
 (segment (start 143.85 95.5) (end 143.45 95.5) (width 0.4572) (layer "B.Cu") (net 1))
 (segment (start 156.65 95.5) (end 143.85 95.5) (width 0.4572) (layer "B.Cu") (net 1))
 (segment (start 143.45 95.5) (end 142.25 96.7) (width 0.4572) (layer "B.Cu") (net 1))
 (segment (start 159.42 110.44) (end 159.15 110.71) (width 0.2032) (layer "F.Cu") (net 24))
 (segment (start 159.15 106.9) (end 158.25 106.9) (width 0.2032) (layer "F.Cu") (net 27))
 (segment (start 159.65 109.94) (end 159.15 109.44) (width 0.2032) (layer "B.Cu") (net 25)))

